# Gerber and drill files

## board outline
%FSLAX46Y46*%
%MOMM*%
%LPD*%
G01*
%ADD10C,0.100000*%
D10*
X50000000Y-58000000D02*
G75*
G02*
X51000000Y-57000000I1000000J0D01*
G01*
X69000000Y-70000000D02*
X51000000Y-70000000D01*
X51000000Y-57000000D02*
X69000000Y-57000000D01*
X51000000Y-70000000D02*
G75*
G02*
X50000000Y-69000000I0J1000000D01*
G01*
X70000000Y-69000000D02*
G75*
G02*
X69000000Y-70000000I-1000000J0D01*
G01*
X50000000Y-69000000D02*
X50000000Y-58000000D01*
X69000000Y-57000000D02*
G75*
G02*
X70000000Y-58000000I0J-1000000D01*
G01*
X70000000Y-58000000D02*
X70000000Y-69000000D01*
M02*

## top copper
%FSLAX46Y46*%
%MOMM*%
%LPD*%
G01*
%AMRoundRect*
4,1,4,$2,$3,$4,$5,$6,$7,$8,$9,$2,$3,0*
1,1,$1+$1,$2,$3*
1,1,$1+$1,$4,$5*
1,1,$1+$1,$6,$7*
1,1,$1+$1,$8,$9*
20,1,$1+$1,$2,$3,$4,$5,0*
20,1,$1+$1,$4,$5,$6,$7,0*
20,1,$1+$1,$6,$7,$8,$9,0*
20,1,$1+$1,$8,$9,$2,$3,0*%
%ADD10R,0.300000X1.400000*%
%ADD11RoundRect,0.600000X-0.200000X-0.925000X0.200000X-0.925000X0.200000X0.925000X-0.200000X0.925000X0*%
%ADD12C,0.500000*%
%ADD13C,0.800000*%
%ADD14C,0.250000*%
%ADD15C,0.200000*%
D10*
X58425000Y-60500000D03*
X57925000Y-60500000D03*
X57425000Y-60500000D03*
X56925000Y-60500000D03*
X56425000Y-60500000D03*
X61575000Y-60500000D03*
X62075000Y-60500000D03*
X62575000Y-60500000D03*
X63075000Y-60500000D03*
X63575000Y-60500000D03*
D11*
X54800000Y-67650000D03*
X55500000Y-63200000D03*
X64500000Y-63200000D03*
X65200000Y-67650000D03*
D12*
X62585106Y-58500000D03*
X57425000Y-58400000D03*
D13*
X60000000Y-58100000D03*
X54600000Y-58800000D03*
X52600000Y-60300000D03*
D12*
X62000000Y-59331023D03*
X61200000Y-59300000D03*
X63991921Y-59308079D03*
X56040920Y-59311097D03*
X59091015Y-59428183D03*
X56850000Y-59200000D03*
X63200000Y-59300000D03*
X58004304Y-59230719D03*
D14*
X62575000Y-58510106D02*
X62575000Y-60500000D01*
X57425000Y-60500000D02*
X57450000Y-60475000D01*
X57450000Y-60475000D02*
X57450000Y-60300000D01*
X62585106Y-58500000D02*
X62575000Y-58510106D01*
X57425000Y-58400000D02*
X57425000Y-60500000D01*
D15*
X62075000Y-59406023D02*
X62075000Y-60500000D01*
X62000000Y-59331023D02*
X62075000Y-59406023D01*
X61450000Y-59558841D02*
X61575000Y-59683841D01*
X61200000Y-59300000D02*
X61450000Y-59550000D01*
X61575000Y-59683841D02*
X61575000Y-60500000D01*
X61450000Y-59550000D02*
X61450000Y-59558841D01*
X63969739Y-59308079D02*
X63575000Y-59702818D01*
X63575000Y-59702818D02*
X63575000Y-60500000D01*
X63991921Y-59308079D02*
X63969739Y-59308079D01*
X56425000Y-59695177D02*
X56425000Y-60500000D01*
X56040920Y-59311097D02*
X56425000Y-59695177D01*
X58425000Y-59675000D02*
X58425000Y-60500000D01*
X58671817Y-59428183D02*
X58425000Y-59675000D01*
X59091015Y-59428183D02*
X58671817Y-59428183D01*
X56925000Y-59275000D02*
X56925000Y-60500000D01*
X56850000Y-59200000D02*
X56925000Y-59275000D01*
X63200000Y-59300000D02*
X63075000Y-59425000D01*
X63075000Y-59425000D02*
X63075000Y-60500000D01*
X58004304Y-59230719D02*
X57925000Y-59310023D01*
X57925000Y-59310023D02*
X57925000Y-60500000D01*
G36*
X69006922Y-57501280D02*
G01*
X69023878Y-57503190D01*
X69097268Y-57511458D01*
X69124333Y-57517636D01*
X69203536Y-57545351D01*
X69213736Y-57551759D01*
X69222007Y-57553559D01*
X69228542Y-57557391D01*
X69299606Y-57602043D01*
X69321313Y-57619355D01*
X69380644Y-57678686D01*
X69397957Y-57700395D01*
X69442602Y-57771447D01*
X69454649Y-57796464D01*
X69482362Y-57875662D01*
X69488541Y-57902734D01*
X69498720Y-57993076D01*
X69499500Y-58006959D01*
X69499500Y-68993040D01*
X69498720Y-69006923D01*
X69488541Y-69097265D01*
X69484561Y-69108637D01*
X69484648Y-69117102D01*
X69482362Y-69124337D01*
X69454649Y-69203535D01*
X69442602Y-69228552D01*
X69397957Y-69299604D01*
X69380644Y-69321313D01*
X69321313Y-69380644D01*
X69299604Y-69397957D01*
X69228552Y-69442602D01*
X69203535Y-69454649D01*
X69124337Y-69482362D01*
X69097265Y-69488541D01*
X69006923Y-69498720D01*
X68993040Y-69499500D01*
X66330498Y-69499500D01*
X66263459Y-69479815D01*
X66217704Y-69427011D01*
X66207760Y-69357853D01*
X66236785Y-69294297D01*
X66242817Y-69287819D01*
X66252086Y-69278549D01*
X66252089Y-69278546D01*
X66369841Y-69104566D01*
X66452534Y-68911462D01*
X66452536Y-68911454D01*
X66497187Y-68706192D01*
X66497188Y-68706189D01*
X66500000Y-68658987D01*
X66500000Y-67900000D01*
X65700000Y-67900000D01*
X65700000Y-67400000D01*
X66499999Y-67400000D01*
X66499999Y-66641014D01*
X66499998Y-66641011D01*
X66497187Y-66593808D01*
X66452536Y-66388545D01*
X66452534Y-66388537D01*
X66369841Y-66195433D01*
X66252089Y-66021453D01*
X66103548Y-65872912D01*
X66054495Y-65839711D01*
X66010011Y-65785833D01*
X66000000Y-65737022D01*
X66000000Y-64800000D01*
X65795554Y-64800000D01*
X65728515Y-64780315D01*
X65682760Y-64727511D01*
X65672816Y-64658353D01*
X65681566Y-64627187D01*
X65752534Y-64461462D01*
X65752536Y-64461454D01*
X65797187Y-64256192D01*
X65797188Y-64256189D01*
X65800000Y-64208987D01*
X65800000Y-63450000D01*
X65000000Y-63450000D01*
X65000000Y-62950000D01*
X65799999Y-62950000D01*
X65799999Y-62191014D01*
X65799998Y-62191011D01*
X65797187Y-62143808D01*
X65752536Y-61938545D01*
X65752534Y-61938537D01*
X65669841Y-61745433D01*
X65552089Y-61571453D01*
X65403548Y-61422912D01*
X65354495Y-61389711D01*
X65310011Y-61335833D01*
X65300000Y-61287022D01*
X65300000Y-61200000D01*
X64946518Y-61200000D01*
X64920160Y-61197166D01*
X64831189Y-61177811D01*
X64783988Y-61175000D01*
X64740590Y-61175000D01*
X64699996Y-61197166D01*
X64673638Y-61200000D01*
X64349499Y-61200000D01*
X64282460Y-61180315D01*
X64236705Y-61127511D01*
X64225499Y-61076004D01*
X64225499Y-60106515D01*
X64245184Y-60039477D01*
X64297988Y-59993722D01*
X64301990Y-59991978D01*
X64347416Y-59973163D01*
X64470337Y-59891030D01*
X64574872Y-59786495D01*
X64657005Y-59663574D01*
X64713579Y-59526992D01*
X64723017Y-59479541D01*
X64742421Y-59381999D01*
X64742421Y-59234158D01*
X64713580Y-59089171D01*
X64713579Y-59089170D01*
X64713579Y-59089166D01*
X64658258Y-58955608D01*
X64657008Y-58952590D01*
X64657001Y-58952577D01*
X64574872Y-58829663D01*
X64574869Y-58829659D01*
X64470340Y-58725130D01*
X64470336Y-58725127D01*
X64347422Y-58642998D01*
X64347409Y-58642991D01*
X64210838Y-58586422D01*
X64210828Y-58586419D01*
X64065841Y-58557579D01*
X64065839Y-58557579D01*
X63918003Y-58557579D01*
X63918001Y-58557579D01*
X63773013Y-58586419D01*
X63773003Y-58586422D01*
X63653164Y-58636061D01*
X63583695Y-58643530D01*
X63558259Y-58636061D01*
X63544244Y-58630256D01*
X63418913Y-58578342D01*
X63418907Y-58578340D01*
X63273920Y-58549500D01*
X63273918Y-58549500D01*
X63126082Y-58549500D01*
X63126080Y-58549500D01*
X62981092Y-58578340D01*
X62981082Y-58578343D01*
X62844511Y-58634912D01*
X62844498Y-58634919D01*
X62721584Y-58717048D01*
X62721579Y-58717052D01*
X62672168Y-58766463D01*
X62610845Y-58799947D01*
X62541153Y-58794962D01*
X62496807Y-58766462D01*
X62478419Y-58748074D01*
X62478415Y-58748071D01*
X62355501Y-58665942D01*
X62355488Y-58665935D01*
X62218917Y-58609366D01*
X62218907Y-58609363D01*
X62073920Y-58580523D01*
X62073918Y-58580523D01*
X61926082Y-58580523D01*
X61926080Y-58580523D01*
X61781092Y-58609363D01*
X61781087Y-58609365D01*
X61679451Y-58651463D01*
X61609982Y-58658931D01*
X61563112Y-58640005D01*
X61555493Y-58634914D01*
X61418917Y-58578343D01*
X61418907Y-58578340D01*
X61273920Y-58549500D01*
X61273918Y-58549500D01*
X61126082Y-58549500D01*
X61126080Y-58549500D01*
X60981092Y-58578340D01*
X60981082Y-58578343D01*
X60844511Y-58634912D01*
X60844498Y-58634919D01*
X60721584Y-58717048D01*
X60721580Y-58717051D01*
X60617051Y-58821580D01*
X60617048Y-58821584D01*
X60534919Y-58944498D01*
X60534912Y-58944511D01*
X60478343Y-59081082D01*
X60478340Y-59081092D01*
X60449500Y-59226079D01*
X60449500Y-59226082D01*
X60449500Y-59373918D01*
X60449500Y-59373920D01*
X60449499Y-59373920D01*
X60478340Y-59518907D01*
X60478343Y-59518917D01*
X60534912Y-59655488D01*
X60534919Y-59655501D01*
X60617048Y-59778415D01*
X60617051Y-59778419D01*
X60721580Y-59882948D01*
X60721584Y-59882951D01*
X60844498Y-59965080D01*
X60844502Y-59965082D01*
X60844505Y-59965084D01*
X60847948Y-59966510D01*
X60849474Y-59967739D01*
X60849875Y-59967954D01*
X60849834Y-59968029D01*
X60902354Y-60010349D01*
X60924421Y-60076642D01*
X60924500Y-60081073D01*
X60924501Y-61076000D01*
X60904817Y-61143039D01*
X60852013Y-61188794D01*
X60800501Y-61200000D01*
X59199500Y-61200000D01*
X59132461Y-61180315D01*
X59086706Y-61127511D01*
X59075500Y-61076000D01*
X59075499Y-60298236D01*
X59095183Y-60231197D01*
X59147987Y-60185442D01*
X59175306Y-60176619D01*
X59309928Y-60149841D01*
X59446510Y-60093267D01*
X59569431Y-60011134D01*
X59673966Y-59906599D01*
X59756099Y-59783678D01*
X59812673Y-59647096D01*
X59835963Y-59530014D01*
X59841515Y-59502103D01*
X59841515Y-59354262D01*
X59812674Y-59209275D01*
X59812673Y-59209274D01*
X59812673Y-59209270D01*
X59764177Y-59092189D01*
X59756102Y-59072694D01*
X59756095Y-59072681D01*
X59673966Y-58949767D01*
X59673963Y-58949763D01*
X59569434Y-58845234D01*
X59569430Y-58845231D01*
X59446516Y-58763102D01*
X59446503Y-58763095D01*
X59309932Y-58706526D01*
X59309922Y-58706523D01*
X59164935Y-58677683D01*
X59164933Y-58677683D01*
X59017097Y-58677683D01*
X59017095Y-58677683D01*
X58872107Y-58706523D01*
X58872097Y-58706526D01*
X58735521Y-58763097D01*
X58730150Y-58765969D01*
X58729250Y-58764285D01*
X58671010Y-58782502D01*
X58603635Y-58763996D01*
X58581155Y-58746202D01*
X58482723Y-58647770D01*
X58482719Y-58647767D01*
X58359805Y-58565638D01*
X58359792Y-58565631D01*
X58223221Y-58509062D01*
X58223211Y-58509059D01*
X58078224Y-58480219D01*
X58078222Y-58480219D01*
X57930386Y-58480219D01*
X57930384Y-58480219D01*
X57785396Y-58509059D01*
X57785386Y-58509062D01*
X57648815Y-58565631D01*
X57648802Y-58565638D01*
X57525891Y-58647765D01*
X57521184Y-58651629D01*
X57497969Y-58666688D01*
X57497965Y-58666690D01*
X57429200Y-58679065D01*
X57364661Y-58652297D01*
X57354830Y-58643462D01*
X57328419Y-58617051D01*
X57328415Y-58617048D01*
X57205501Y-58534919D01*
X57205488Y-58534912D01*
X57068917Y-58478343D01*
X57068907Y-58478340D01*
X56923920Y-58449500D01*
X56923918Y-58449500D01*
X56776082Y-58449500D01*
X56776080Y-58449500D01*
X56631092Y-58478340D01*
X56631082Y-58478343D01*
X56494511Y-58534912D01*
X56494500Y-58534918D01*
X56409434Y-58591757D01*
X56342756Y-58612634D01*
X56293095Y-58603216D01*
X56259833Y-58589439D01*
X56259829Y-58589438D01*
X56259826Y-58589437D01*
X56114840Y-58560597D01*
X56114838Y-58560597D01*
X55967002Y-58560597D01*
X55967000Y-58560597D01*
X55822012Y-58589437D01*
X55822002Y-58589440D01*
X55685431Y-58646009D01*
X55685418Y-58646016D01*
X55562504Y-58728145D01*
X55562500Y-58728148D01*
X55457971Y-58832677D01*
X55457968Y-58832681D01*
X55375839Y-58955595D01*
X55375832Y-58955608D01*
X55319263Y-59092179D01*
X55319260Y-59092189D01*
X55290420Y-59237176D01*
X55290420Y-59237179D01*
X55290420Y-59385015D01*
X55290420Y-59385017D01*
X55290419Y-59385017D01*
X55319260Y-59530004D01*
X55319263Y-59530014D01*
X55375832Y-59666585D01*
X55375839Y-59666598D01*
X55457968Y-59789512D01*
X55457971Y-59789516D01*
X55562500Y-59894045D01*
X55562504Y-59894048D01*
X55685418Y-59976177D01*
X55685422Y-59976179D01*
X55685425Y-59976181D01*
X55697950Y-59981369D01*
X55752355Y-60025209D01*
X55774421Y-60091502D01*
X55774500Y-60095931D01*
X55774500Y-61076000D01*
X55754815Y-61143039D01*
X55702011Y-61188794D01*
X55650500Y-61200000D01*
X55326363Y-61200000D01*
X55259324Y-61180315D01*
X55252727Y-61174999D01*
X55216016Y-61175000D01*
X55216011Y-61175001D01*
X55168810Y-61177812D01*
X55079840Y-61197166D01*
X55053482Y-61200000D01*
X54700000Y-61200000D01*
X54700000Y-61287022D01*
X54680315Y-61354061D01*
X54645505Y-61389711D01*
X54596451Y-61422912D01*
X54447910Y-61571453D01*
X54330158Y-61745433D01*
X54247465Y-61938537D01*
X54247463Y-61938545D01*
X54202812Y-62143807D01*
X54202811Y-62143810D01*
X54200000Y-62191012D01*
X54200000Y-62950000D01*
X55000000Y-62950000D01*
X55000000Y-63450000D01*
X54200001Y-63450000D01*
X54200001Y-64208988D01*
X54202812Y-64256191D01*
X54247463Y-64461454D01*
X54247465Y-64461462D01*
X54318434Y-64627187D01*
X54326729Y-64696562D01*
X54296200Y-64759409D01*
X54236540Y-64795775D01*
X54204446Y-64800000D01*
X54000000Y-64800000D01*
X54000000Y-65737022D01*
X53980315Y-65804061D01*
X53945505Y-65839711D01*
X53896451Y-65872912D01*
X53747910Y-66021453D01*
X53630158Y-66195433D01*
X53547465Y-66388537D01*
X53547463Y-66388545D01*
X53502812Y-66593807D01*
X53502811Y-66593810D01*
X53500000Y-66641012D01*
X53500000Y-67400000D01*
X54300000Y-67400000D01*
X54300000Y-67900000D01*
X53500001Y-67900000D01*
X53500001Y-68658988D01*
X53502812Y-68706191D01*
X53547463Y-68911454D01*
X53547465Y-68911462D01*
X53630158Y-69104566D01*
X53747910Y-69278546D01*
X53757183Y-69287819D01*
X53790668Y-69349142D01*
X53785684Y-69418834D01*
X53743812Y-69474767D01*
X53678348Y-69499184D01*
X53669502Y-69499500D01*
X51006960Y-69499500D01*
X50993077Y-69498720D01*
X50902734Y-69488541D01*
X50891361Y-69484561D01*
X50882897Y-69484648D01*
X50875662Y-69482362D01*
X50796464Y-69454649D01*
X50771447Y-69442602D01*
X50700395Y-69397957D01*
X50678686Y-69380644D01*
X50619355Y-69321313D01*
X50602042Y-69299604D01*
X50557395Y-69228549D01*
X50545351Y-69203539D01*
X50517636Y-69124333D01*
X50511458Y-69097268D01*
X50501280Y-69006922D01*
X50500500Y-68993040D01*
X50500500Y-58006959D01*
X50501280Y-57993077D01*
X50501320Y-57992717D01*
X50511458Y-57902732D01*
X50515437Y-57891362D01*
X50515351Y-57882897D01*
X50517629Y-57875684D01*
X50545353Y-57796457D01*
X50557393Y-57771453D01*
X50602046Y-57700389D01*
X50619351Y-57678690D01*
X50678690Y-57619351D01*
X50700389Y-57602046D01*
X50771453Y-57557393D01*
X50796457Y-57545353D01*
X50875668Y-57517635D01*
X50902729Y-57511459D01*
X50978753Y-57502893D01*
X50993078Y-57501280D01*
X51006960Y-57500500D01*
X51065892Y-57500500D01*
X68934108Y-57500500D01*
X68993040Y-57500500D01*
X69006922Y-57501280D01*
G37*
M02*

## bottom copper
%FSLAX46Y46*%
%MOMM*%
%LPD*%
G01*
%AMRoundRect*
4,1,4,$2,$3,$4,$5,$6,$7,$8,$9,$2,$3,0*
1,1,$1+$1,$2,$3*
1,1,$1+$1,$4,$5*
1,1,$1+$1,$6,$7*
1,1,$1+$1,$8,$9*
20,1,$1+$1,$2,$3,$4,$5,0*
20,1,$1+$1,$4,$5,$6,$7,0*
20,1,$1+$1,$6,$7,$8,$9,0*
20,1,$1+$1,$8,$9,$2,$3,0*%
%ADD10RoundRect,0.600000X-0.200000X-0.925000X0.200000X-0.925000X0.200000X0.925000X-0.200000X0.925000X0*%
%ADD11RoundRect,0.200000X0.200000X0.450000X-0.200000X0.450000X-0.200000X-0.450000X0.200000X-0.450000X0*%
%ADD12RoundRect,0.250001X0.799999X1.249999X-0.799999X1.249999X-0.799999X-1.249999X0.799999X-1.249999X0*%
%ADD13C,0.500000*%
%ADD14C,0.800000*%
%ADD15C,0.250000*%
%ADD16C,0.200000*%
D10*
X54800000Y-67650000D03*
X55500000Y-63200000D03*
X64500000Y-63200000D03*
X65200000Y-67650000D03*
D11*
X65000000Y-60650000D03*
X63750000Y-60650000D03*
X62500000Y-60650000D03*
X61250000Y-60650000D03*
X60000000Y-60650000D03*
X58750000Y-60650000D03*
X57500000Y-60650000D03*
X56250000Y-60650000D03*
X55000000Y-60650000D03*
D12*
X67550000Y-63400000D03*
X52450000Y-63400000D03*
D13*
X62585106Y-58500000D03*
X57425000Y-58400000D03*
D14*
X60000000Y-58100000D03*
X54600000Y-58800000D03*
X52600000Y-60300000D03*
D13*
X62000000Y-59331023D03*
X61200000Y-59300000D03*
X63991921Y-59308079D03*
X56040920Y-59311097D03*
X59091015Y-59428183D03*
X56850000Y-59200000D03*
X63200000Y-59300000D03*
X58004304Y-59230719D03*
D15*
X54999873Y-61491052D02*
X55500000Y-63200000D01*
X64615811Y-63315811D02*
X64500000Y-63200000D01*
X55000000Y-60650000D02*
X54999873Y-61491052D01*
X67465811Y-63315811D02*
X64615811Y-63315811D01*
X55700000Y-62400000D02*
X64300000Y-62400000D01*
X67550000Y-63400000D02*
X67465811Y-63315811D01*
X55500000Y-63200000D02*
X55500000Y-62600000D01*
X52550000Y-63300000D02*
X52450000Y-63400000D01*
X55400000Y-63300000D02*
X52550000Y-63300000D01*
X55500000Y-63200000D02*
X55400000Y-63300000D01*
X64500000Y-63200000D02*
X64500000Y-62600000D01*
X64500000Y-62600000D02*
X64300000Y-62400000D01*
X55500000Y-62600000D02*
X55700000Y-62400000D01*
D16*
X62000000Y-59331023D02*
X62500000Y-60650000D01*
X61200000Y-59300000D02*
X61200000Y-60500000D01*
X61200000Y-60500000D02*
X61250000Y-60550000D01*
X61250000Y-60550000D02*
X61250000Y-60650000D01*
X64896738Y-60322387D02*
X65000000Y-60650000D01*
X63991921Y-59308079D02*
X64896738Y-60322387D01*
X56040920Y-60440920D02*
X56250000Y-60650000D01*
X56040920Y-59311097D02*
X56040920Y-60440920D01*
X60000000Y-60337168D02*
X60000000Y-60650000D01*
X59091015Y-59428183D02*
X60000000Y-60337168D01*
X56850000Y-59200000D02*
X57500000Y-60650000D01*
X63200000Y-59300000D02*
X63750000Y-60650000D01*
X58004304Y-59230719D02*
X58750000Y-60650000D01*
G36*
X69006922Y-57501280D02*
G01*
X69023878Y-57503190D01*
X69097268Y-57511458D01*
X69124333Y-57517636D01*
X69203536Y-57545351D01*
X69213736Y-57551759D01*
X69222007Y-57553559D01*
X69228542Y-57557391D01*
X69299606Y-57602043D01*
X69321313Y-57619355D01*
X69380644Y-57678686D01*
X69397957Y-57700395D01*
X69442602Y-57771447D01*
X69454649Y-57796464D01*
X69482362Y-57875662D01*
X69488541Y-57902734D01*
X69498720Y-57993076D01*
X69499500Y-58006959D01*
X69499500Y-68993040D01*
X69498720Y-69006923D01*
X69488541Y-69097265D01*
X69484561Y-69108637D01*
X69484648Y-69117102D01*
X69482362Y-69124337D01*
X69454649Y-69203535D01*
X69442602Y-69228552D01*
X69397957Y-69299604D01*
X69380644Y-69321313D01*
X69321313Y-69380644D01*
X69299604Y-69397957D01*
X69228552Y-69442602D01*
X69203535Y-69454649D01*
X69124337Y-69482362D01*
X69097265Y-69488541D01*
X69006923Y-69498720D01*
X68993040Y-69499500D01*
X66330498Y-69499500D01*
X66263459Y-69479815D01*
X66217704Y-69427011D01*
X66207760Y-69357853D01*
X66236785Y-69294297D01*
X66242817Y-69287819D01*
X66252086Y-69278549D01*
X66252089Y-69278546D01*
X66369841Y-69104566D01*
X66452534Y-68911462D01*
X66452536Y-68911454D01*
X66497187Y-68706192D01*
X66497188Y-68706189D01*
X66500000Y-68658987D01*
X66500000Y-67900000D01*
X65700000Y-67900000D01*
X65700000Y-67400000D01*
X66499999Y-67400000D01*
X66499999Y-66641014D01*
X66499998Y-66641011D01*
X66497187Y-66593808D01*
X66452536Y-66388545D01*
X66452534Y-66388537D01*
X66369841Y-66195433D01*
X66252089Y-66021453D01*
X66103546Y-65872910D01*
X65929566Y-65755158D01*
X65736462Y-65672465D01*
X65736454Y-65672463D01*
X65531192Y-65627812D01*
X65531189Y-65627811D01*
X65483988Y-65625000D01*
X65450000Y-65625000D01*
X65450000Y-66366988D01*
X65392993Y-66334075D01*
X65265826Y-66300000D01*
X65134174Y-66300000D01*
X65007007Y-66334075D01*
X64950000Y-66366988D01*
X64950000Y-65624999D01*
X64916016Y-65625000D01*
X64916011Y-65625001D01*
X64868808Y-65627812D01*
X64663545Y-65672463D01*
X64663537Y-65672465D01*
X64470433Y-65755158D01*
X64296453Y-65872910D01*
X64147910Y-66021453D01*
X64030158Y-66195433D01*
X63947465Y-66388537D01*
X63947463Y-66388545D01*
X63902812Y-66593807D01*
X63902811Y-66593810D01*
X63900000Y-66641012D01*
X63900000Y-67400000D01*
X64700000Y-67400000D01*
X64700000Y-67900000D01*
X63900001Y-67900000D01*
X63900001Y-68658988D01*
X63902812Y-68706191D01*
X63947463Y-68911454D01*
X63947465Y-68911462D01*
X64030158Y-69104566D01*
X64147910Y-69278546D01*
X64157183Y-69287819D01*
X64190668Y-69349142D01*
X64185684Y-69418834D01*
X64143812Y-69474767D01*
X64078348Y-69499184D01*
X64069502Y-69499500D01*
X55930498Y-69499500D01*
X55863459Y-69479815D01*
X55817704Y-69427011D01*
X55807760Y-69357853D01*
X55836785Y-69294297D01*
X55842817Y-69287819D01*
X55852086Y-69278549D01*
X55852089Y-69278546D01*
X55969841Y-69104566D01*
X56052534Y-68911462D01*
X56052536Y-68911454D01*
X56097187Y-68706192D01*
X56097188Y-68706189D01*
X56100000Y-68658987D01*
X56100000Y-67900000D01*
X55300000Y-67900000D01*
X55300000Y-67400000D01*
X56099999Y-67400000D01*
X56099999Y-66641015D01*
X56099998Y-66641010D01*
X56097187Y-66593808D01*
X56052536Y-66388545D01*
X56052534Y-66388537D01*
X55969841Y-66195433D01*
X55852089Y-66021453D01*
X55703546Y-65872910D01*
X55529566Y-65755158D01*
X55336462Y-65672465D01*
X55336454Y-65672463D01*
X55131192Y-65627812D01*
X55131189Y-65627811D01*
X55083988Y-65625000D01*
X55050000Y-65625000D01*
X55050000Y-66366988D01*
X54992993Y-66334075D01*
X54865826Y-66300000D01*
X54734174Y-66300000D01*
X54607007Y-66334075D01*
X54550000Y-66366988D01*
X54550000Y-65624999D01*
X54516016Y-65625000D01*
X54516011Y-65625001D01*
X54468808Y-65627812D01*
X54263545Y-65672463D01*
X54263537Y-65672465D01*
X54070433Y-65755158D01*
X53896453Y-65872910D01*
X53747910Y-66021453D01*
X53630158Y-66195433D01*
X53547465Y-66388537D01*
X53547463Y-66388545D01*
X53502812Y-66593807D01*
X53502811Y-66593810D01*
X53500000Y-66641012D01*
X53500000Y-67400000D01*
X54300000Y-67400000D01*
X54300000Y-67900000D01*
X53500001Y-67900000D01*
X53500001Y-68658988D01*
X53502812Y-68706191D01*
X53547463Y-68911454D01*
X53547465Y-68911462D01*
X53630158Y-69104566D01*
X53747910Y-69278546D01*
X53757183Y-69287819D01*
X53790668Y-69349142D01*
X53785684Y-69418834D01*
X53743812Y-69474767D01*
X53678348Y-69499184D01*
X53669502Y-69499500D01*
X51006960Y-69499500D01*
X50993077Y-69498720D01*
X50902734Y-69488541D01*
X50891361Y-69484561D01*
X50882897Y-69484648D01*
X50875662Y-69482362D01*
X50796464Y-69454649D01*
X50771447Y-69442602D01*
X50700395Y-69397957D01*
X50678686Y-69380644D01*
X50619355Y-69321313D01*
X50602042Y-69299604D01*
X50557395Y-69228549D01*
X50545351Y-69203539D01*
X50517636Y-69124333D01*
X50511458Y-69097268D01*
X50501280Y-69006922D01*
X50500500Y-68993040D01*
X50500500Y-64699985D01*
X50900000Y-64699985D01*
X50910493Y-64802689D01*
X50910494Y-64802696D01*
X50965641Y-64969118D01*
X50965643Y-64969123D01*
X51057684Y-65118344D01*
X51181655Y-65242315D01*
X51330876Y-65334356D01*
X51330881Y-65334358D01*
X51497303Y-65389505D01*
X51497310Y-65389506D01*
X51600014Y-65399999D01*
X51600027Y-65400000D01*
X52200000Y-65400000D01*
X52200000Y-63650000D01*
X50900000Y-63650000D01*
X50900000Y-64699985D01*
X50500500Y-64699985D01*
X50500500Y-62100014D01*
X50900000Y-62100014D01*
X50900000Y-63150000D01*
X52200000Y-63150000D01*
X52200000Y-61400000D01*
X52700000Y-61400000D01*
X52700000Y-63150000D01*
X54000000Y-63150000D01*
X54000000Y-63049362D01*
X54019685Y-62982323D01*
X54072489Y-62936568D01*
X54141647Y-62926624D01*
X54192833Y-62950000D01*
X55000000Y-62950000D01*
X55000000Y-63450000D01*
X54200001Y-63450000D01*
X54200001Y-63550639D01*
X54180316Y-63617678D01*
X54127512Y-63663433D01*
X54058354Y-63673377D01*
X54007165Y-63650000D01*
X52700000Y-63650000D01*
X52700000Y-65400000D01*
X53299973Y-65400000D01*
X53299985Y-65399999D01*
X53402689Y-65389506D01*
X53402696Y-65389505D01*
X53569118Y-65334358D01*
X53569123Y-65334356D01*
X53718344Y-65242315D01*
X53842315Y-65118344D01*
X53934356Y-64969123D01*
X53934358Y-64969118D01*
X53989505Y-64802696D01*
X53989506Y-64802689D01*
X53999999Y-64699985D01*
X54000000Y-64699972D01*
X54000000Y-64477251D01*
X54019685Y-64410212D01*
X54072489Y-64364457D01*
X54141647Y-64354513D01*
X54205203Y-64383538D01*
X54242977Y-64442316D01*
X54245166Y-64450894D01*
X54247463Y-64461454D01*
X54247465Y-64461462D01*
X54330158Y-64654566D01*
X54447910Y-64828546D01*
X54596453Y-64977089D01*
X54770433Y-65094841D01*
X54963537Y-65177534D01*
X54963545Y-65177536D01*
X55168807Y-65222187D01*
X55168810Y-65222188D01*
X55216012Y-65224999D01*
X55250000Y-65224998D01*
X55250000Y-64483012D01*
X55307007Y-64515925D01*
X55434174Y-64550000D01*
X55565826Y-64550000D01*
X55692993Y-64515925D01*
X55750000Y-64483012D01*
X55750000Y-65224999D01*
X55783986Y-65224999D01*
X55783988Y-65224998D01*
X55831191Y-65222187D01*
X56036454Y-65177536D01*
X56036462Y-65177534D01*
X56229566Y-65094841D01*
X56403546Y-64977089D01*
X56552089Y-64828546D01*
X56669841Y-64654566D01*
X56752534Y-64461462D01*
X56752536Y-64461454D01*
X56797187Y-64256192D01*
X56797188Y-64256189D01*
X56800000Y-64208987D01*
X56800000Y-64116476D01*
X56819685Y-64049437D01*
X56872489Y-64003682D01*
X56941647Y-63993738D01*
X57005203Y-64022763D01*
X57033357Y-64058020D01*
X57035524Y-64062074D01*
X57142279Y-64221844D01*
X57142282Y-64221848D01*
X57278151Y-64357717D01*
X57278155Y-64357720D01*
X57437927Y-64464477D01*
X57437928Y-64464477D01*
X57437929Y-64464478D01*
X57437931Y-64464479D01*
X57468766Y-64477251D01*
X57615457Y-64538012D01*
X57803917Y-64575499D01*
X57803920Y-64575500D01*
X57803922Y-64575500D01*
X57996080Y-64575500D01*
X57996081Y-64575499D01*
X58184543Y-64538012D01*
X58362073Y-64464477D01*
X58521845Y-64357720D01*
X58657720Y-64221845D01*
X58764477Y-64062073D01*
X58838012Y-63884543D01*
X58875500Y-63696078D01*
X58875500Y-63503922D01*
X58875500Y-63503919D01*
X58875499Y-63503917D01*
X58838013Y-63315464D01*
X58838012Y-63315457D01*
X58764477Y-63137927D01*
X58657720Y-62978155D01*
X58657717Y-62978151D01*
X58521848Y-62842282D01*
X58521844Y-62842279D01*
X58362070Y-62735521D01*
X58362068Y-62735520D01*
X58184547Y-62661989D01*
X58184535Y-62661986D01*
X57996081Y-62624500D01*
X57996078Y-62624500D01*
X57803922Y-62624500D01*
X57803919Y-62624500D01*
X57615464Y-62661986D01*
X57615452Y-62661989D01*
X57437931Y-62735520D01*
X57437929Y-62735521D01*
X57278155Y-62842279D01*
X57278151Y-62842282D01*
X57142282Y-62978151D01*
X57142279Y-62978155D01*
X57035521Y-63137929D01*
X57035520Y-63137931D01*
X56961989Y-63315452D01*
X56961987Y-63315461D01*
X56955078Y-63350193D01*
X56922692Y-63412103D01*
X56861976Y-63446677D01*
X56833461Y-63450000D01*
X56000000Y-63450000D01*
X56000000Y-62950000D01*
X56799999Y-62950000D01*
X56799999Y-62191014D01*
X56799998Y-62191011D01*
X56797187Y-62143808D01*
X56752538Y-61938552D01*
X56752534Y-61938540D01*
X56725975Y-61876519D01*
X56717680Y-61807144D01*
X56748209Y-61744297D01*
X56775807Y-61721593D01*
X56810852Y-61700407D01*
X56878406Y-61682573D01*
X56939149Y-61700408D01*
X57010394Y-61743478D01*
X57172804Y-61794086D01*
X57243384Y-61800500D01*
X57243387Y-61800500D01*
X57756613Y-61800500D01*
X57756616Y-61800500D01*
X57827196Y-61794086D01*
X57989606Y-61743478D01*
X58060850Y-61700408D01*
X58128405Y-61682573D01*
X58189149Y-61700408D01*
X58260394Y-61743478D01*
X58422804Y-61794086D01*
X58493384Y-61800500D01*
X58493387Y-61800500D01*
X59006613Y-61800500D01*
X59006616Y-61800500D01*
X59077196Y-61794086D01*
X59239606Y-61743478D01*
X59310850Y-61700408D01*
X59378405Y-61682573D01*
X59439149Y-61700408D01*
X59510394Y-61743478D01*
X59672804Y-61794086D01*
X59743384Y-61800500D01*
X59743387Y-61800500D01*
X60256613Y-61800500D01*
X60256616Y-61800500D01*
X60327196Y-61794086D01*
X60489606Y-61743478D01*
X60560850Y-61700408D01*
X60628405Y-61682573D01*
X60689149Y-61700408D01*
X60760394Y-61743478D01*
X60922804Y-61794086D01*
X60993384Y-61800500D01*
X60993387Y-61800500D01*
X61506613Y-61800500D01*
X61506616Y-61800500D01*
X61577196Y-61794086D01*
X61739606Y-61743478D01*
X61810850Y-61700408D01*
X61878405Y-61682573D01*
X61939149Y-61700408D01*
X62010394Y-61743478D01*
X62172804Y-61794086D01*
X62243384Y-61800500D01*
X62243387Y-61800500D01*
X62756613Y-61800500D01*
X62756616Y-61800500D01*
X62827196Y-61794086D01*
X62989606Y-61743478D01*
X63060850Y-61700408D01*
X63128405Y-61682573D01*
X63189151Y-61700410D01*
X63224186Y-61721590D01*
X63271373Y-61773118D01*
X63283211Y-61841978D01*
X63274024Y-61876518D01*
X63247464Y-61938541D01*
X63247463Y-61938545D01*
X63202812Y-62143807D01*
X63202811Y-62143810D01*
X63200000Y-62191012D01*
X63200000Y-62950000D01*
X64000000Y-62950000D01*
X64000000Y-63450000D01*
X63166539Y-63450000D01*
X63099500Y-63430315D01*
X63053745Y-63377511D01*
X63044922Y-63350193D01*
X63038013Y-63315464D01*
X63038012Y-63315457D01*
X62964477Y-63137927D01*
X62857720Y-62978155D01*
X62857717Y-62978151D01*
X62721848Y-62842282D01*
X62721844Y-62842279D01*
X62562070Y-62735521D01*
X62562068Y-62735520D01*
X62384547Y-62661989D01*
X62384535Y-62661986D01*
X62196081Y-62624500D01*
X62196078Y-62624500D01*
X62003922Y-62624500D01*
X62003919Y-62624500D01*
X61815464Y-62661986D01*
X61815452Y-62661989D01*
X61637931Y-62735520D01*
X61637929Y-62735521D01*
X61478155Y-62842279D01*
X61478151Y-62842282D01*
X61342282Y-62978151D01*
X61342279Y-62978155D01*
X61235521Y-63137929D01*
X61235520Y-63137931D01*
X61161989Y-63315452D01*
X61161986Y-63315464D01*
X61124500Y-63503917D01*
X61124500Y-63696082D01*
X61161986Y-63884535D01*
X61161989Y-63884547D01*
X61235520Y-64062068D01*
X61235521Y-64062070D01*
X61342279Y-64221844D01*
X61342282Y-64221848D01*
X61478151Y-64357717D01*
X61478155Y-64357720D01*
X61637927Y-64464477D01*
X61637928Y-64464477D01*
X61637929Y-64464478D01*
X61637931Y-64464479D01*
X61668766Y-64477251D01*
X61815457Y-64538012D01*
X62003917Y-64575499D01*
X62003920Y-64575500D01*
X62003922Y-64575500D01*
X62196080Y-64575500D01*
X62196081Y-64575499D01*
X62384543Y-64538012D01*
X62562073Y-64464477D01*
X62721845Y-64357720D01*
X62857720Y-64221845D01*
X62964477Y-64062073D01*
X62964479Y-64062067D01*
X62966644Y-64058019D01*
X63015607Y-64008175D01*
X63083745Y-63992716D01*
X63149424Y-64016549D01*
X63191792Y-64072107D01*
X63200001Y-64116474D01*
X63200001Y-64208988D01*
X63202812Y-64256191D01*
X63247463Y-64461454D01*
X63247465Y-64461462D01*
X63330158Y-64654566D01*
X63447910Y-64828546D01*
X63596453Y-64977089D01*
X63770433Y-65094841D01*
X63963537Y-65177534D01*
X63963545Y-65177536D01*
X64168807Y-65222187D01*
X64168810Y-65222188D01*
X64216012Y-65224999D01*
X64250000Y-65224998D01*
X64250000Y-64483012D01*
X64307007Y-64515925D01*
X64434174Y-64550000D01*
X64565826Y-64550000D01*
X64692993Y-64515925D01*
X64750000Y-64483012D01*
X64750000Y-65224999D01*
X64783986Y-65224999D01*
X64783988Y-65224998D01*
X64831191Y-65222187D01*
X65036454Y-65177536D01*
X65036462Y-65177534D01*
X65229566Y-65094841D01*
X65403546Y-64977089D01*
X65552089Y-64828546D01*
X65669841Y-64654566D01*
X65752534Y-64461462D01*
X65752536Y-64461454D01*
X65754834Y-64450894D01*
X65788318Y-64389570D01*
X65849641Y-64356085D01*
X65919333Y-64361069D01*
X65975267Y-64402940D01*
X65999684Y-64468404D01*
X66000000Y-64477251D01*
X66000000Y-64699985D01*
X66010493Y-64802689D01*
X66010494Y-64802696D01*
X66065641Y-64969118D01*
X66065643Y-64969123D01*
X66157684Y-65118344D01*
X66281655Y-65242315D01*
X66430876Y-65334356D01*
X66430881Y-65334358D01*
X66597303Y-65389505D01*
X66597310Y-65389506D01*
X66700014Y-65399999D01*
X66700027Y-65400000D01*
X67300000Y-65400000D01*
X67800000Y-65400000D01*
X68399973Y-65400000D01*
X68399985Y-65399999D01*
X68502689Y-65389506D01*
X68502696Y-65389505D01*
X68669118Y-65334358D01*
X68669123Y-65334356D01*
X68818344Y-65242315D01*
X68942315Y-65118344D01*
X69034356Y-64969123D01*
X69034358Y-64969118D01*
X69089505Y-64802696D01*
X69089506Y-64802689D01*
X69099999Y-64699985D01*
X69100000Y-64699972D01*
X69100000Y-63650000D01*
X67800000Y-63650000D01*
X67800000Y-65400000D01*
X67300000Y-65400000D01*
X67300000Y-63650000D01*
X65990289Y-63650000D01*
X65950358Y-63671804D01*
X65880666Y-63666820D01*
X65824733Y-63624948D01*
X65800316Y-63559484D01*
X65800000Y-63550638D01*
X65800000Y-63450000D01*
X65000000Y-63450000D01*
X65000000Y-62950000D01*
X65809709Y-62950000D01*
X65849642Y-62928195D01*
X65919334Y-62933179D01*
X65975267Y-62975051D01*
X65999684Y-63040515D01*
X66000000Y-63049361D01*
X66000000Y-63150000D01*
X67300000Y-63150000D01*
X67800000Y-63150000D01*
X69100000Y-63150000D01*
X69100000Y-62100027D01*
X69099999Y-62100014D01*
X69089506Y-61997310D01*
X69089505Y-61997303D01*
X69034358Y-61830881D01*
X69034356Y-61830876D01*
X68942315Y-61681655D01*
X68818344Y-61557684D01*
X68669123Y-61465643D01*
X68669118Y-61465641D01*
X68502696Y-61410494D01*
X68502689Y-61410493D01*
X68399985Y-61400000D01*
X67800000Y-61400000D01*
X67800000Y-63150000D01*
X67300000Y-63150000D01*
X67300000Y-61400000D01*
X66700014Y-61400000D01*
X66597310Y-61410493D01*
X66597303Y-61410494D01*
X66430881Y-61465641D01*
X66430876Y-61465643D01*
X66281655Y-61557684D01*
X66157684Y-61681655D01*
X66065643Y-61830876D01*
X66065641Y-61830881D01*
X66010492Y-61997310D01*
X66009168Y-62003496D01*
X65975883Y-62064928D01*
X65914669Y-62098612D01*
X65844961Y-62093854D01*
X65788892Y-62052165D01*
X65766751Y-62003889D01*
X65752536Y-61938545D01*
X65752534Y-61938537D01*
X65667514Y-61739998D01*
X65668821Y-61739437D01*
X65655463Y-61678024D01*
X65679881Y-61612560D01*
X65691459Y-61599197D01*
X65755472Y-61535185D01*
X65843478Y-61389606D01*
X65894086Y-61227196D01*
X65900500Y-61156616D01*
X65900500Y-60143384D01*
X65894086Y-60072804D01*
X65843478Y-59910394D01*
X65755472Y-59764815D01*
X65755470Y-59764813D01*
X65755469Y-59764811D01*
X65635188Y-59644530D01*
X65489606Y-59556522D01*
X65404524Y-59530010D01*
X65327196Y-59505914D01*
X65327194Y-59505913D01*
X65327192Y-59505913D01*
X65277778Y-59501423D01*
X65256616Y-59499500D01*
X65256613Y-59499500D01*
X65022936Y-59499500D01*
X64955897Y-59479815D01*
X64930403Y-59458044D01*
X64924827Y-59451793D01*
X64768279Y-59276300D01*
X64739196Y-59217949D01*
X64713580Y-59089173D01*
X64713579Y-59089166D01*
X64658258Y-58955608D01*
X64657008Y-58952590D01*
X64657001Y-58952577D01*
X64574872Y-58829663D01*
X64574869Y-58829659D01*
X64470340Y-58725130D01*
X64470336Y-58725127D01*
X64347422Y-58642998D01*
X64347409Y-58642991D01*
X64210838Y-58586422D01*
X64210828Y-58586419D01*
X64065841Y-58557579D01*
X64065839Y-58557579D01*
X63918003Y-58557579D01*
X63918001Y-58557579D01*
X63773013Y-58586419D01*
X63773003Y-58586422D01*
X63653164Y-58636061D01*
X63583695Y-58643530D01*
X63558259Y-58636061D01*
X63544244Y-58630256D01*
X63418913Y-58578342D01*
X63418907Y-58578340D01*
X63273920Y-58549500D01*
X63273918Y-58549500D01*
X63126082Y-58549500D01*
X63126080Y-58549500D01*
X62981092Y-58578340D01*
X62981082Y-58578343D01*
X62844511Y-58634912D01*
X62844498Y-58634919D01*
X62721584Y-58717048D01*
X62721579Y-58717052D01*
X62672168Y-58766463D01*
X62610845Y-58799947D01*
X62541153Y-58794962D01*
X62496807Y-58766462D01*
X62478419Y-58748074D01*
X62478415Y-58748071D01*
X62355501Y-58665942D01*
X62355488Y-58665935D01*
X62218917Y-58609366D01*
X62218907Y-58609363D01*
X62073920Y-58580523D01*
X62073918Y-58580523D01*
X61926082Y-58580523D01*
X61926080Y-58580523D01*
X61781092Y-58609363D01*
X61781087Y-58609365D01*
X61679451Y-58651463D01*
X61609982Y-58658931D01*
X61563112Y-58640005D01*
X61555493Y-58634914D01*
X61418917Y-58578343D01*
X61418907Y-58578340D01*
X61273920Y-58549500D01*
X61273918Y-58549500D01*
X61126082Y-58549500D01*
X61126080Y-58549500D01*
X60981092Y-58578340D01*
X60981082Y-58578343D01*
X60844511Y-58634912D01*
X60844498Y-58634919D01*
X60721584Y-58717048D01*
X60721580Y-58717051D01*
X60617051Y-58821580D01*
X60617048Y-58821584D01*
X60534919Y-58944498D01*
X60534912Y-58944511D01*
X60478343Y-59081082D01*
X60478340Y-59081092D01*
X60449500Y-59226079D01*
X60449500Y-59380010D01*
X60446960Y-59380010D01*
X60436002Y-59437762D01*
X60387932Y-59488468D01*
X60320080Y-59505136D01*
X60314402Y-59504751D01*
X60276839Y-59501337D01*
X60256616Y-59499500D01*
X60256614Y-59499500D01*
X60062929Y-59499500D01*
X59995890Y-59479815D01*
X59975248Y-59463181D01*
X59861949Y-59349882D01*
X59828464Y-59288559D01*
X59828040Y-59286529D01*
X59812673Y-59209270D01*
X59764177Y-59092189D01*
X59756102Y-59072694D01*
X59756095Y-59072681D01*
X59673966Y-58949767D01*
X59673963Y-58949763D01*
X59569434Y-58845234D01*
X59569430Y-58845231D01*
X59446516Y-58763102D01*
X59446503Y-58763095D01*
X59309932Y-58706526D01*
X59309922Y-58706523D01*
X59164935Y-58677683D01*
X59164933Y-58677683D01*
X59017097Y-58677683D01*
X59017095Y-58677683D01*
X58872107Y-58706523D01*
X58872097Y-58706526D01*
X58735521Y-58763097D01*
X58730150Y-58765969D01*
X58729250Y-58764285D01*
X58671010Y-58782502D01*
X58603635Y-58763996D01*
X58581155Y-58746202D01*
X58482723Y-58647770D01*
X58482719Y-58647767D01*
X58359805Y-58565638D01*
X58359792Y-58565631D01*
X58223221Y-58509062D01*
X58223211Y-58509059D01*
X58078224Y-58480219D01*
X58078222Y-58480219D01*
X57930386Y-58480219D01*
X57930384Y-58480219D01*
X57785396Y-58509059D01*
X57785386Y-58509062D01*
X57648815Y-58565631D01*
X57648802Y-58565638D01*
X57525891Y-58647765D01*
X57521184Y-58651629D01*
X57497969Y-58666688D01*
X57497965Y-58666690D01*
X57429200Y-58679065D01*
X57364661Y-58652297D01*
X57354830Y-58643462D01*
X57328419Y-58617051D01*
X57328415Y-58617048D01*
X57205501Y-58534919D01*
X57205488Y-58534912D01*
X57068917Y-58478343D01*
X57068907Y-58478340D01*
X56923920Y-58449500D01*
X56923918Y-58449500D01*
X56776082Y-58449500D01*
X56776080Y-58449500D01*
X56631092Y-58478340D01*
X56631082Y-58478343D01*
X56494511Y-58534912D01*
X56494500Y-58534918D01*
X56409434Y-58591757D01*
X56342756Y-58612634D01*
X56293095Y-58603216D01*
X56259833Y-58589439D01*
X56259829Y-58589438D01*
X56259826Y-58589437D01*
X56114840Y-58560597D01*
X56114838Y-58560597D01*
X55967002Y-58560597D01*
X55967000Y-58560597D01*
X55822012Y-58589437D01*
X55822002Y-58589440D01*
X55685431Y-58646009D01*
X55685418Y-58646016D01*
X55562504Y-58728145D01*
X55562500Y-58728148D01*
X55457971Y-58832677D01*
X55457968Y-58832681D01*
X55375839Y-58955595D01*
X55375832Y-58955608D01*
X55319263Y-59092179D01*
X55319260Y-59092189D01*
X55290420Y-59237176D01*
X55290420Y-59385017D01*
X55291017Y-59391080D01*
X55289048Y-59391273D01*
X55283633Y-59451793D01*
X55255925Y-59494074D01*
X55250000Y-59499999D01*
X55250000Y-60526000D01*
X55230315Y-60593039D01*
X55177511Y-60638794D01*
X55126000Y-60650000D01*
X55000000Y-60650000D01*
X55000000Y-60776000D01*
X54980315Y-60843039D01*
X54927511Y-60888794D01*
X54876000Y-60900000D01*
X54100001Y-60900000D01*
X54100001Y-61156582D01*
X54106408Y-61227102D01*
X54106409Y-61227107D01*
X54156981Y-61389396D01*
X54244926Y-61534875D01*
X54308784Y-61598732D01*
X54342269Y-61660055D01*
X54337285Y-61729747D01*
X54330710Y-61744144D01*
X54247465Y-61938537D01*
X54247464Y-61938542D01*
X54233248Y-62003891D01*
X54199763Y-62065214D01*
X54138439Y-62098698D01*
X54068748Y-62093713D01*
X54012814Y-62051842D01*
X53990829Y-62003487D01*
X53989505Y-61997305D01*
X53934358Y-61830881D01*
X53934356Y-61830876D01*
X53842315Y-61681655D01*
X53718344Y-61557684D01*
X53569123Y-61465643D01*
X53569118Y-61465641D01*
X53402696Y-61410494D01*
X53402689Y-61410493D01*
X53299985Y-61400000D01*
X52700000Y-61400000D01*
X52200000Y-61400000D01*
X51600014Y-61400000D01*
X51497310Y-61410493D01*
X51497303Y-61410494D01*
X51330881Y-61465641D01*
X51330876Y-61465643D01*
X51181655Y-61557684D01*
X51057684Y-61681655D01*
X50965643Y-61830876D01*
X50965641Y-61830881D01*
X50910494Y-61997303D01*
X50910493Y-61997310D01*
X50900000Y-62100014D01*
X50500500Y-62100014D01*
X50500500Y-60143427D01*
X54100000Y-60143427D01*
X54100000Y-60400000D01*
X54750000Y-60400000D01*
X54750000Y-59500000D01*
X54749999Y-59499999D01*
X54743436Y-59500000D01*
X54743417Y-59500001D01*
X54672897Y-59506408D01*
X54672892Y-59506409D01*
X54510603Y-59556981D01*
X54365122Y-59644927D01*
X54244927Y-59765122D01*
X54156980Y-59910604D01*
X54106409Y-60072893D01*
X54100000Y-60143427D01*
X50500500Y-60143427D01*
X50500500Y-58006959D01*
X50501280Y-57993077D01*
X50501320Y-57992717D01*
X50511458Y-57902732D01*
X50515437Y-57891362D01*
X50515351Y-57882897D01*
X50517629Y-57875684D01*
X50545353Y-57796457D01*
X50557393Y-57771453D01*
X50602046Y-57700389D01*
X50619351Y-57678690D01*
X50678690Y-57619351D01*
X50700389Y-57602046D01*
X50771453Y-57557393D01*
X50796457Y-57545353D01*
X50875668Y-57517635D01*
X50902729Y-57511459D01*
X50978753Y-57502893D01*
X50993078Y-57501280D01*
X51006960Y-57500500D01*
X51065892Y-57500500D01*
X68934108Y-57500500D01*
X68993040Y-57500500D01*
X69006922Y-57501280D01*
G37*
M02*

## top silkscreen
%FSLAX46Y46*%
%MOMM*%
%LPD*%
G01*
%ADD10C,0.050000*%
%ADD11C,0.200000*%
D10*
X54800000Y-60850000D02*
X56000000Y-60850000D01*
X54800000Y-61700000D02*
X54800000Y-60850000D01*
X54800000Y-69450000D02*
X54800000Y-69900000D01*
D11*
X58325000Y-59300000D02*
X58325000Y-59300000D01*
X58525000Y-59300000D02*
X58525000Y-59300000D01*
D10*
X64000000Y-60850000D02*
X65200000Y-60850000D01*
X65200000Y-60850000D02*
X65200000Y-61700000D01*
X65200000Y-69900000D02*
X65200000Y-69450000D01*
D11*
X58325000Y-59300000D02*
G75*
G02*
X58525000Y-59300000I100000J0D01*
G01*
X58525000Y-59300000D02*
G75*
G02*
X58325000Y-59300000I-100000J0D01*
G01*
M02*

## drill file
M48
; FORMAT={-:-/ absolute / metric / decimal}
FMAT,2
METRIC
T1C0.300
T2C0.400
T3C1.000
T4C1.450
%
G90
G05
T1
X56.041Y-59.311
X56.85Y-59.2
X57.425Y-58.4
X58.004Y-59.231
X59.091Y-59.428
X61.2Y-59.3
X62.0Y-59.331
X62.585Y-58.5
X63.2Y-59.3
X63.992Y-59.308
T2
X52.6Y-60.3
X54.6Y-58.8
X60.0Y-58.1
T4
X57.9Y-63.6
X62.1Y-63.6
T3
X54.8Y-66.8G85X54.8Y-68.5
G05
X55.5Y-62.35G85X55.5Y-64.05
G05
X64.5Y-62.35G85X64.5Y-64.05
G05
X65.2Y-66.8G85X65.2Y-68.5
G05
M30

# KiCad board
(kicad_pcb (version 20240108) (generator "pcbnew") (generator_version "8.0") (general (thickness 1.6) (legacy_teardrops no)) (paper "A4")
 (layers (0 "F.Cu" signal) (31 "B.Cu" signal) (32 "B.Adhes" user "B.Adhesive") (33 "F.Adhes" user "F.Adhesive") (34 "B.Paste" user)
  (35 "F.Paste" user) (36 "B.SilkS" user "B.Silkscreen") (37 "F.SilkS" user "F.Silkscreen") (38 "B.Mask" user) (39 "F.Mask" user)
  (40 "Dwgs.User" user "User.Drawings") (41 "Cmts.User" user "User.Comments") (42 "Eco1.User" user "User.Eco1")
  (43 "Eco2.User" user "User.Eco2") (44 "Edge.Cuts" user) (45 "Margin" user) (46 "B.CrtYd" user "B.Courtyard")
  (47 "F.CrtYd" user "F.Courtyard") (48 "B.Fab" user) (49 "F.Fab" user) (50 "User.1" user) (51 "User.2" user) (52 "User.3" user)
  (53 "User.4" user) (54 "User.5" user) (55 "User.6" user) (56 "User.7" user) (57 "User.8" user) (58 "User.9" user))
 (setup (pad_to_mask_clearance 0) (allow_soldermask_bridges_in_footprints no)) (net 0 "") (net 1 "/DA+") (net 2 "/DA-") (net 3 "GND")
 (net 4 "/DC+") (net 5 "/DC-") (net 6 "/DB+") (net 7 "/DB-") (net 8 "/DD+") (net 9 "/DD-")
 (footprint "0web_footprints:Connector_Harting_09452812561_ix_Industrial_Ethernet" (layer "F.Cu") (at 60 70)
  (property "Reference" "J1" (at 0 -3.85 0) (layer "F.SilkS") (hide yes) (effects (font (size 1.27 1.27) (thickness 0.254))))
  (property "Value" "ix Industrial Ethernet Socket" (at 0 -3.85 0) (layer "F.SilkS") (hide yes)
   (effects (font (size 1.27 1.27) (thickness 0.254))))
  (fp_line (start -5.2 -9.15) (end -4 -9.15) (stroke (width 0.05) (type solid)) (layer "F.SilkS"))
  (fp_line (start -5.2 -8.3) (end -5.2 -9.15) (stroke (width 0.05) (type solid)) (layer "F.SilkS"))
  (fp_line (start -5.2 -0.55) (end -5.2 -0.1) (stroke (width 0.05) (type solid)) (layer "F.SilkS"))
  (fp_line (start -1.675 -10.7) (end -1.675 -10.7) (stroke (width 0.2) (type solid)) (layer "F.SilkS"))
  (fp_line (start -1.475 -10.7) (end -1.475 -10.7) (stroke (width 0.2) (type solid)) (layer "F.SilkS"))
  (fp_line (start 4 -9.15) (end 5.2 -9.15) (stroke (width 0.05) (type solid)) (layer "F.SilkS"))
  (fp_line (start 5.2 -9.15) (end 5.2 -8.3) (stroke (width 0.05) (type solid)) (layer "F.SilkS"))
  (fp_line (start 5.2 -0.1) (end 5.2 -0.55) (stroke (width 0.05) (type solid)) (layer "F.SilkS"))
  (fp_arc (start -1.675 -10.7) (mid -1.575 -10.8) (end -1.475 -10.7) (stroke (width 0.2) (type solid)) (layer "F.SilkS"))
  (fp_arc (start -1.475 -10.7) (mid -1.575 -10.6) (end -1.675 -10.7) (stroke (width 0.2) (type solid)) (layer "F.SilkS"))
  (pad "" np_thru_hole circle (at -2.1 -6.4) (size 1.45 1.45) (drill 1.45) (layers "*.Cu" "*.Mask"))
  (pad "" np_thru_hole circle (at 2.1 -6.4) (size 1.45 1.45) (drill 1.45) (layers "*.Cu" "*.Mask"))
  (pad "1" smd rect (at -1.575 -9.5) (size 0.3 1.4) (layers "F.Cu" "F.Paste" "F.Mask") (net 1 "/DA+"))
  (pad "2" smd rect (at -2.075 -9.5) (size 0.3 1.4) (layers "F.Cu" "F.Paste" "F.Mask") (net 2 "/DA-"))
  (pad "3" smd rect (at -2.575 -9.5) (size 0.3 1.4) (layers "F.Cu" "F.Paste" "F.Mask") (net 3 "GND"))
  (pad "4" smd rect (at -3.075 -9.5) (size 0.3 1.4) (layers "F.Cu" "F.Paste" "F.Mask") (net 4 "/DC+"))
  (pad "5" smd rect (at -3.575 -9.5) (size 0.3 1.4) (layers "F.Cu" "F.Paste" "F.Mask") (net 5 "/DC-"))
  (pad "6" smd rect (at 1.575 -9.5) (size 0.3 1.4) (layers "F.Cu" "F.Paste" "F.Mask") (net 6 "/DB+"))
  (pad "7" smd rect (at 2.075 -9.5) (size 0.3 1.4) (layers "F.Cu" "F.Paste" "F.Mask") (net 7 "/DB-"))
  (pad "8" smd rect (at 2.575 -9.5) (size 0.3 1.4) (layers "F.Cu" "F.Paste" "F.Mask") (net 3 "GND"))
  (pad "9" smd rect (at 3.075 -9.5) (size 0.3 1.4) (layers "F.Cu" "F.Paste" "F.Mask") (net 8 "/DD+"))
  (pad "10" smd rect (at 3.575 -9.5) (size 0.3 1.4) (layers "F.Cu" "F.Paste" "F.Mask") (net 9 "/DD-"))
  (pad "11" thru_hole roundrect (at -5.2 -2.35) (size 1.6 3.05) (drill oval 1 2.7) (layers "*.Cu" "*.Mask") (remove_unused_layers no)
   (roundrect_rratio 0.375) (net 3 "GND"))
  (pad "11" thru_hole roundrect (at -4.5 -6.8) (size 1.6 3.05) (drill oval 1 2.7) (layers "*.Cu" "*.Mask") (remove_unused_layers no)
   (roundrect_rratio 0.375) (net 3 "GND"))
  (pad "11" thru_hole roundrect (at 4.5 -6.8) (size 1.6 3.05) (drill oval 1 2.7) (layers "*.Cu" "*.Mask") (remove_unused_layers no)
   (roundrect_rratio 0.375) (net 3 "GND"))
  (pad "11" thru_hole roundrect (at 5.2 -2.35) (size 1.6 3.05) (drill oval 1 2.7) (layers "*.Cu" "*.Mask") (remove_unused_layers no)
   (roundrect_rratio 0.375) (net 3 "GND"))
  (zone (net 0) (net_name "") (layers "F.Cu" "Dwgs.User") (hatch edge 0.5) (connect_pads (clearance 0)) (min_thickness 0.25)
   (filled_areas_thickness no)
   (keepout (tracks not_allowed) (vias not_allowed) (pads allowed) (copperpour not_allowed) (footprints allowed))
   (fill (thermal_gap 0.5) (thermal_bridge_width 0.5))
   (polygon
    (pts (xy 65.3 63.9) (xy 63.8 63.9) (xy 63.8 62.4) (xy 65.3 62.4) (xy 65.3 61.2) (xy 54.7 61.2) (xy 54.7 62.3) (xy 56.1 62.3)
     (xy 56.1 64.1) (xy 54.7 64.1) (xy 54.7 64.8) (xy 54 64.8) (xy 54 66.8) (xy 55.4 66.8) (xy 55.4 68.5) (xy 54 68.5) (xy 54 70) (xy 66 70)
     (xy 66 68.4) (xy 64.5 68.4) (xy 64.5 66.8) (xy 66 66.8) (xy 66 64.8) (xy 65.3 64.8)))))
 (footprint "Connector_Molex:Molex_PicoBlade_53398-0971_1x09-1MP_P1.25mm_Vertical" (layer "B.Cu") (at 60 61.9 180)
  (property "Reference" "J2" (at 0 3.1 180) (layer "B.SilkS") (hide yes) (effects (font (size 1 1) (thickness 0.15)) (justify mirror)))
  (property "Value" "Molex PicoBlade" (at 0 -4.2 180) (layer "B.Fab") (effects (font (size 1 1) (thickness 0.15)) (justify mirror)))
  (pad "1" smd roundrect (at -5 1.25 180) (size 0.8 1.3) (layers "B.Cu" "B.Paste" "B.Mask") (roundrect_rratio 0.25) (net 9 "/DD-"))
  (pad "2" smd roundrect (at -3.75 1.25 180) (size 0.8 1.3) (layers "B.Cu" "B.Paste" "B.Mask") (roundrect_rratio 0.25) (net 8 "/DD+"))
  (pad "3" smd roundrect (at -2.5 1.25 180) (size 0.8 1.3) (layers "B.Cu" "B.Paste" "B.Mask") (roundrect_rratio 0.25) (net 7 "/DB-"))
  (pad "4" smd roundrect (at -1.25 1.25 180) (size 0.8 1.3) (layers "B.Cu" "B.Paste" "B.Mask") (roundrect_rratio 0.25) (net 6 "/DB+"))
  (pad "5" smd roundrect (at 0 1.25 180) (size 0.8 1.3) (layers "B.Cu" "B.Paste" "B.Mask") (roundrect_rratio 0.25) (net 1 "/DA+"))
  (pad "6" smd roundrect (at 1.25 1.25 180) (size 0.8 1.3) (layers "B.Cu" "B.Paste" "B.Mask") (roundrect_rratio 0.25) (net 2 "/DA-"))
  (pad "7" smd roundrect (at 2.5 1.25 180) (size 0.8 1.3) (layers "B.Cu" "B.Paste" "B.Mask") (roundrect_rratio 0.25) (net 4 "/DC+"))
  (pad "8" smd roundrect (at 3.75 1.25 180) (size 0.8 1.3) (layers "B.Cu" "B.Paste" "B.Mask") (roundrect_rratio 0.25) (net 5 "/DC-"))
  (pad "9" smd roundrect (at 5 1.25 180) (size 0.8 1.3) (layers "B.Cu" "B.Paste" "B.Mask") (roundrect_rratio 0.25) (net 3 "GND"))
  (pad "MP" smd roundrect (at -7.55 -1.5 180) (size 2.1 3) (layers "B.Cu" "B.Paste" "B.Mask") (roundrect_rratio 0.1190480952) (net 3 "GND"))
  (pad "MP" smd roundrect (at 7.55 -1.5 180) (size 2.1 3) (layers "B.Cu" "B.Paste" "B.Mask") (roundrect_rratio 0.1190480952) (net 3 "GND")))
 (gr_arc (start 50 58) (mid 50.292893 57.292893) (end 51 57) (stroke (width 0.1) (type default)) (layer "Edge.Cuts"))
 (gr_line (start 69 70) (end 51 70) (stroke (width 0.1) (type default)) (layer "Edge.Cuts"))
 (gr_line (start 51 57) (end 69 57) (stroke (width 0.1) (type default)) (layer "Edge.Cuts"))
 (gr_arc (start 51 70) (mid 50.292893 69.707107) (end 50 69) (stroke (width 0.1) (type default)) (layer "Edge.Cuts"))
 (gr_arc (start 70 69) (mid 69.707107 69.707107) (end 69 70) (stroke (width 0.1) (type default)) (layer "Edge.Cuts"))
 (gr_line (start 50 69) (end 50 58) (stroke (width 0.1) (type default)) (layer "Edge.Cuts"))
 (gr_arc (start 69 57) (mid 69.707107 57.292893) (end 70 58) (stroke (width 0.1) (type default)) (layer "Edge.Cuts"))
 (gr_line (start 70 58) (end 70 69) (stroke (width 0.1) (type default)) (layer "Edge.Cuts"))
 (segment (start 62.575 58.510106) (end 62.575 60.5) (width 0.25) (layer "F.Cu") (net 3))
 (segment (start 57.425 60.5) (end 57.45 60.475) (width 0.25) (layer "F.Cu") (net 3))
 (segment (start 57.45 60.475) (end 57.45 60.3) (width 0.25) (layer "F.Cu") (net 3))
 (segment (start 62.585106 58.5) (end 62.575 58.510106) (width 0.25) (layer "F.Cu") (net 3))
 (segment (start 57.425 58.4) (end 57.425 60.5) (width 0.25) (layer "F.Cu") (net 3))
 (via (at 62.585106 58.5) (size 0.5) (drill 0.3) (layers "F.Cu" "B.Cu") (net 3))
 (via (at 57.425 58.4) (size 0.5) (drill 0.3) (layers "F.Cu" "B.Cu") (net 3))
 (via (at 60 58.1) (size 0.8) (drill 0.4) (layers "F.Cu" "B.Cu") (free yes) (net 3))
 (via (at 54.6 58.8) (size 0.8) (drill 0.4) (layers "F.Cu" "B.Cu") (free yes) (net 3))
 (via (at 52.6 60.3) (size 0.8) (drill 0.4) (layers "F.Cu" "B.Cu") (free yes) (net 3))
 (segment (start 54.999873 61.491052) (end 55.5 63.2) (width 0.25) (layer "B.Cu") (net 3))
 (segment (start 64.615811 63.315811) (end 64.5 63.2) (width 0.25) (layer "B.Cu") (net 3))
 (segment (start 55 60.65) (end 54.999873 61.491052) (width 0.25) (layer "B.Cu") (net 3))
 (segment (start 67.465811 63.315811) (end 64.615811 63.315811) (width 0.25) (layer "B.Cu") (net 3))
 (segment (start 55.7 62.4) (end 64.3 62.4) (width 0.25) (layer "B.Cu") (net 3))
 (segment (start 67.55 63.4) (end 67.465811 63.315811) (width 0.25) (layer "B.Cu") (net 3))
 (segment (start 55.5 63.2) (end 55.5 62.6) (width 0.25) (layer "B.Cu") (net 3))
 (segment (start 52.55 63.3) (end 52.45 63.4) (width 0.25) (layer "B.Cu") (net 3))
 (segment (start 55.4 63.3) (end 52.55 63.3) (width 0.25) (layer "B.Cu") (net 3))
 (segment (start 55.5 63.2) (end 55.4 63.3) (width 0.25) (layer "B.Cu") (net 3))
 (segment (start 64.5 63.2) (end 64.5 62.6) (width 0.25) (layer "B.Cu") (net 3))
 (segment (start 64.5 62.6) (end 64.3 62.4) (width 0.25) (layer "B.Cu") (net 3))
 (segment (start 55.5 62.6) (end 55.7 62.4) (width 0.25) (layer "B.Cu") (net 3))
 (segment (start 62.075 59.406023) (end 62.075 60.5) (width 0.2) (layer "F.Cu") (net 7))
 (segment (start 62 59.331023) (end 62.075 59.406023) (width 0.2) (layer "F.Cu") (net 7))
 (via (at 62 59.331023) (size 0.5) (drill 0.3) (layers "F.Cu" "B.Cu") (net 7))
 (segment (start 62 59.331023) (end 62.5 60.65) (width 0.2) (layer "B.Cu") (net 7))
 (segment (start 61.45 59.558841) (end 61.575 59.683841) (width 0.2) (layer "F.Cu") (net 6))
 (segment (start 61.2 59.3) (end 61.45 59.55) (width 0.2) (layer "F.Cu") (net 6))
 (segment (start 61.575 59.683841) (end 61.575 60.5) (width 0.2) (layer "F.Cu") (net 6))
 (segment (start 61.45 59.55) (end 61.45 59.558841) (width 0.2) (layer "F.Cu") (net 6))
 (via (at 61.2 59.3) (size 0.5) (drill 0.3) (layers "F.Cu" "B.Cu") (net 6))
 (segment (start 61.2 59.3) (end 61.2 60.5) (width 0.2) (layer "B.Cu") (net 6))
 (segment (start 61.2 60.5) (end 61.25 60.55) (width 0.2) (layer "B.Cu") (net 6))
 (segment (start 61.25 60.55) (end 61.25 60.65) (width 0.2) (layer "B.Cu") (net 6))
 (segment (start 63.969739 59.308079) (end 63.575 59.702818) (width 0.2) (layer "F.Cu") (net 9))
 (segment (start 63.575 59.702818) (end 63.575 60.5) (width 0.2) (layer "F.Cu") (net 9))
 (segment (start 63.991921 59.308079) (end 63.969739 59.308079) (width 0.2) (layer "F.Cu") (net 9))
 (via (at 63.991921 59.308079) (size 0.5) (drill 0.3) (layers "F.Cu" "B.Cu") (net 9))
 (segment (start 64.896738 60.322387) (end 65 60.65) (width 0.2) (layer "B.Cu") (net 9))
 (segment (start 63.991921 59.308079) (end 64.896738 60.322387) (width 0.2) (layer "B.Cu") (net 9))
 (segment (start 56.425 59.695177) (end 56.425 60.5) (width 0.2) (layer "F.Cu") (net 5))
 (segment (start 56.04092 59.311097) (end 56.425 59.695177) (width 0.2) (layer "F.Cu") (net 5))
 (via (at 56.04092 59.311097) (size 0.5) (drill 0.3) (layers "F.Cu" "B.Cu") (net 5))
 (segment (start 56.04092 60.44092) (end 56.25 60.65) (width 0.2) (layer "B.Cu") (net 5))
 (segment (start 56.04092 59.311097) (end 56.04092 60.44092) (width 0.2) (layer "B.Cu") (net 5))
 (segment (start 58.425 59.675) (end 58.425 60.5) (width 0.2) (layer "F.Cu") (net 1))
 (segment (start 58.671817 59.428183) (end 58.425 59.675) (width 0.2) (layer "F.Cu") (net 1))
 (segment (start 59.091015 59.428183) (end 58.671817 59.428183) (width 0.2) (layer "F.Cu") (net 1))
 (via (at 59.091015 59.428183) (size 0.5) (drill 0.3) (layers "F.Cu" "B.Cu") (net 1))
 (segment (start 60 60.337168) (end 60 60.65) (width 0.2) (layer "B.Cu") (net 1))
 (segment (start 59.091015 59.428183) (end 60 60.337168) (width 0.2) (layer "B.Cu") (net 1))
 (segment (start 56.925 59.275) (end 56.925 60.5) (width 0.2) (layer "F.Cu") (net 4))
 (segment (start 56.85 59.2) (end 56.925 59.275) (width 0.2) (layer "F.Cu") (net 4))
 (via (at 56.85 59.2) (size 0.5) (drill 0.3) (layers "F.Cu" "B.Cu") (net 4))
 (segment (start 56.85 59.2) (end 57.5 60.65) (width 0.2) (layer "B.Cu") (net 4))
 (segment (start 63.2 59.3) (end 63.075 59.425) (width 0.2) (layer "F.Cu") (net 8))
 (segment (start 63.075 59.425) (end 63.075 60.5) (width 0.2) (layer "F.Cu") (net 8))
 (via (at 63.2 59.3) (size 0.5) (drill 0.3) (layers "F.Cu" "B.Cu") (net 8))
 (segment (start 63.2 59.3) (end 63.75 60.65) (width 0.2) (layer "B.Cu") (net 8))
 (segment (start 58.004304 59.230719) (end 57.925 59.310023) (width 0.2) (layer "F.Cu") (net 2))
 (segment (start 57.925 59.310023) (end 57.925 60.5) (width 0.2) (layer "F.Cu") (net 2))
 (via (at 58.004304 59.230719) (size 0.5) (drill 0.3) (layers "F.Cu" "B.Cu") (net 2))
 (segment (start 58.004304 59.230719) (end 58.75 60.65) (width 0.2) (layer "B.Cu") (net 2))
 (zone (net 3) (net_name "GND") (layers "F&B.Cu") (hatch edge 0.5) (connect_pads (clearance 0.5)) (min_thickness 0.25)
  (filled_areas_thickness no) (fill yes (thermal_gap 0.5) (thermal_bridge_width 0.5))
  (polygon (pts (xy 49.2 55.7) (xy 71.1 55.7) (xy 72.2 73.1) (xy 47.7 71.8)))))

